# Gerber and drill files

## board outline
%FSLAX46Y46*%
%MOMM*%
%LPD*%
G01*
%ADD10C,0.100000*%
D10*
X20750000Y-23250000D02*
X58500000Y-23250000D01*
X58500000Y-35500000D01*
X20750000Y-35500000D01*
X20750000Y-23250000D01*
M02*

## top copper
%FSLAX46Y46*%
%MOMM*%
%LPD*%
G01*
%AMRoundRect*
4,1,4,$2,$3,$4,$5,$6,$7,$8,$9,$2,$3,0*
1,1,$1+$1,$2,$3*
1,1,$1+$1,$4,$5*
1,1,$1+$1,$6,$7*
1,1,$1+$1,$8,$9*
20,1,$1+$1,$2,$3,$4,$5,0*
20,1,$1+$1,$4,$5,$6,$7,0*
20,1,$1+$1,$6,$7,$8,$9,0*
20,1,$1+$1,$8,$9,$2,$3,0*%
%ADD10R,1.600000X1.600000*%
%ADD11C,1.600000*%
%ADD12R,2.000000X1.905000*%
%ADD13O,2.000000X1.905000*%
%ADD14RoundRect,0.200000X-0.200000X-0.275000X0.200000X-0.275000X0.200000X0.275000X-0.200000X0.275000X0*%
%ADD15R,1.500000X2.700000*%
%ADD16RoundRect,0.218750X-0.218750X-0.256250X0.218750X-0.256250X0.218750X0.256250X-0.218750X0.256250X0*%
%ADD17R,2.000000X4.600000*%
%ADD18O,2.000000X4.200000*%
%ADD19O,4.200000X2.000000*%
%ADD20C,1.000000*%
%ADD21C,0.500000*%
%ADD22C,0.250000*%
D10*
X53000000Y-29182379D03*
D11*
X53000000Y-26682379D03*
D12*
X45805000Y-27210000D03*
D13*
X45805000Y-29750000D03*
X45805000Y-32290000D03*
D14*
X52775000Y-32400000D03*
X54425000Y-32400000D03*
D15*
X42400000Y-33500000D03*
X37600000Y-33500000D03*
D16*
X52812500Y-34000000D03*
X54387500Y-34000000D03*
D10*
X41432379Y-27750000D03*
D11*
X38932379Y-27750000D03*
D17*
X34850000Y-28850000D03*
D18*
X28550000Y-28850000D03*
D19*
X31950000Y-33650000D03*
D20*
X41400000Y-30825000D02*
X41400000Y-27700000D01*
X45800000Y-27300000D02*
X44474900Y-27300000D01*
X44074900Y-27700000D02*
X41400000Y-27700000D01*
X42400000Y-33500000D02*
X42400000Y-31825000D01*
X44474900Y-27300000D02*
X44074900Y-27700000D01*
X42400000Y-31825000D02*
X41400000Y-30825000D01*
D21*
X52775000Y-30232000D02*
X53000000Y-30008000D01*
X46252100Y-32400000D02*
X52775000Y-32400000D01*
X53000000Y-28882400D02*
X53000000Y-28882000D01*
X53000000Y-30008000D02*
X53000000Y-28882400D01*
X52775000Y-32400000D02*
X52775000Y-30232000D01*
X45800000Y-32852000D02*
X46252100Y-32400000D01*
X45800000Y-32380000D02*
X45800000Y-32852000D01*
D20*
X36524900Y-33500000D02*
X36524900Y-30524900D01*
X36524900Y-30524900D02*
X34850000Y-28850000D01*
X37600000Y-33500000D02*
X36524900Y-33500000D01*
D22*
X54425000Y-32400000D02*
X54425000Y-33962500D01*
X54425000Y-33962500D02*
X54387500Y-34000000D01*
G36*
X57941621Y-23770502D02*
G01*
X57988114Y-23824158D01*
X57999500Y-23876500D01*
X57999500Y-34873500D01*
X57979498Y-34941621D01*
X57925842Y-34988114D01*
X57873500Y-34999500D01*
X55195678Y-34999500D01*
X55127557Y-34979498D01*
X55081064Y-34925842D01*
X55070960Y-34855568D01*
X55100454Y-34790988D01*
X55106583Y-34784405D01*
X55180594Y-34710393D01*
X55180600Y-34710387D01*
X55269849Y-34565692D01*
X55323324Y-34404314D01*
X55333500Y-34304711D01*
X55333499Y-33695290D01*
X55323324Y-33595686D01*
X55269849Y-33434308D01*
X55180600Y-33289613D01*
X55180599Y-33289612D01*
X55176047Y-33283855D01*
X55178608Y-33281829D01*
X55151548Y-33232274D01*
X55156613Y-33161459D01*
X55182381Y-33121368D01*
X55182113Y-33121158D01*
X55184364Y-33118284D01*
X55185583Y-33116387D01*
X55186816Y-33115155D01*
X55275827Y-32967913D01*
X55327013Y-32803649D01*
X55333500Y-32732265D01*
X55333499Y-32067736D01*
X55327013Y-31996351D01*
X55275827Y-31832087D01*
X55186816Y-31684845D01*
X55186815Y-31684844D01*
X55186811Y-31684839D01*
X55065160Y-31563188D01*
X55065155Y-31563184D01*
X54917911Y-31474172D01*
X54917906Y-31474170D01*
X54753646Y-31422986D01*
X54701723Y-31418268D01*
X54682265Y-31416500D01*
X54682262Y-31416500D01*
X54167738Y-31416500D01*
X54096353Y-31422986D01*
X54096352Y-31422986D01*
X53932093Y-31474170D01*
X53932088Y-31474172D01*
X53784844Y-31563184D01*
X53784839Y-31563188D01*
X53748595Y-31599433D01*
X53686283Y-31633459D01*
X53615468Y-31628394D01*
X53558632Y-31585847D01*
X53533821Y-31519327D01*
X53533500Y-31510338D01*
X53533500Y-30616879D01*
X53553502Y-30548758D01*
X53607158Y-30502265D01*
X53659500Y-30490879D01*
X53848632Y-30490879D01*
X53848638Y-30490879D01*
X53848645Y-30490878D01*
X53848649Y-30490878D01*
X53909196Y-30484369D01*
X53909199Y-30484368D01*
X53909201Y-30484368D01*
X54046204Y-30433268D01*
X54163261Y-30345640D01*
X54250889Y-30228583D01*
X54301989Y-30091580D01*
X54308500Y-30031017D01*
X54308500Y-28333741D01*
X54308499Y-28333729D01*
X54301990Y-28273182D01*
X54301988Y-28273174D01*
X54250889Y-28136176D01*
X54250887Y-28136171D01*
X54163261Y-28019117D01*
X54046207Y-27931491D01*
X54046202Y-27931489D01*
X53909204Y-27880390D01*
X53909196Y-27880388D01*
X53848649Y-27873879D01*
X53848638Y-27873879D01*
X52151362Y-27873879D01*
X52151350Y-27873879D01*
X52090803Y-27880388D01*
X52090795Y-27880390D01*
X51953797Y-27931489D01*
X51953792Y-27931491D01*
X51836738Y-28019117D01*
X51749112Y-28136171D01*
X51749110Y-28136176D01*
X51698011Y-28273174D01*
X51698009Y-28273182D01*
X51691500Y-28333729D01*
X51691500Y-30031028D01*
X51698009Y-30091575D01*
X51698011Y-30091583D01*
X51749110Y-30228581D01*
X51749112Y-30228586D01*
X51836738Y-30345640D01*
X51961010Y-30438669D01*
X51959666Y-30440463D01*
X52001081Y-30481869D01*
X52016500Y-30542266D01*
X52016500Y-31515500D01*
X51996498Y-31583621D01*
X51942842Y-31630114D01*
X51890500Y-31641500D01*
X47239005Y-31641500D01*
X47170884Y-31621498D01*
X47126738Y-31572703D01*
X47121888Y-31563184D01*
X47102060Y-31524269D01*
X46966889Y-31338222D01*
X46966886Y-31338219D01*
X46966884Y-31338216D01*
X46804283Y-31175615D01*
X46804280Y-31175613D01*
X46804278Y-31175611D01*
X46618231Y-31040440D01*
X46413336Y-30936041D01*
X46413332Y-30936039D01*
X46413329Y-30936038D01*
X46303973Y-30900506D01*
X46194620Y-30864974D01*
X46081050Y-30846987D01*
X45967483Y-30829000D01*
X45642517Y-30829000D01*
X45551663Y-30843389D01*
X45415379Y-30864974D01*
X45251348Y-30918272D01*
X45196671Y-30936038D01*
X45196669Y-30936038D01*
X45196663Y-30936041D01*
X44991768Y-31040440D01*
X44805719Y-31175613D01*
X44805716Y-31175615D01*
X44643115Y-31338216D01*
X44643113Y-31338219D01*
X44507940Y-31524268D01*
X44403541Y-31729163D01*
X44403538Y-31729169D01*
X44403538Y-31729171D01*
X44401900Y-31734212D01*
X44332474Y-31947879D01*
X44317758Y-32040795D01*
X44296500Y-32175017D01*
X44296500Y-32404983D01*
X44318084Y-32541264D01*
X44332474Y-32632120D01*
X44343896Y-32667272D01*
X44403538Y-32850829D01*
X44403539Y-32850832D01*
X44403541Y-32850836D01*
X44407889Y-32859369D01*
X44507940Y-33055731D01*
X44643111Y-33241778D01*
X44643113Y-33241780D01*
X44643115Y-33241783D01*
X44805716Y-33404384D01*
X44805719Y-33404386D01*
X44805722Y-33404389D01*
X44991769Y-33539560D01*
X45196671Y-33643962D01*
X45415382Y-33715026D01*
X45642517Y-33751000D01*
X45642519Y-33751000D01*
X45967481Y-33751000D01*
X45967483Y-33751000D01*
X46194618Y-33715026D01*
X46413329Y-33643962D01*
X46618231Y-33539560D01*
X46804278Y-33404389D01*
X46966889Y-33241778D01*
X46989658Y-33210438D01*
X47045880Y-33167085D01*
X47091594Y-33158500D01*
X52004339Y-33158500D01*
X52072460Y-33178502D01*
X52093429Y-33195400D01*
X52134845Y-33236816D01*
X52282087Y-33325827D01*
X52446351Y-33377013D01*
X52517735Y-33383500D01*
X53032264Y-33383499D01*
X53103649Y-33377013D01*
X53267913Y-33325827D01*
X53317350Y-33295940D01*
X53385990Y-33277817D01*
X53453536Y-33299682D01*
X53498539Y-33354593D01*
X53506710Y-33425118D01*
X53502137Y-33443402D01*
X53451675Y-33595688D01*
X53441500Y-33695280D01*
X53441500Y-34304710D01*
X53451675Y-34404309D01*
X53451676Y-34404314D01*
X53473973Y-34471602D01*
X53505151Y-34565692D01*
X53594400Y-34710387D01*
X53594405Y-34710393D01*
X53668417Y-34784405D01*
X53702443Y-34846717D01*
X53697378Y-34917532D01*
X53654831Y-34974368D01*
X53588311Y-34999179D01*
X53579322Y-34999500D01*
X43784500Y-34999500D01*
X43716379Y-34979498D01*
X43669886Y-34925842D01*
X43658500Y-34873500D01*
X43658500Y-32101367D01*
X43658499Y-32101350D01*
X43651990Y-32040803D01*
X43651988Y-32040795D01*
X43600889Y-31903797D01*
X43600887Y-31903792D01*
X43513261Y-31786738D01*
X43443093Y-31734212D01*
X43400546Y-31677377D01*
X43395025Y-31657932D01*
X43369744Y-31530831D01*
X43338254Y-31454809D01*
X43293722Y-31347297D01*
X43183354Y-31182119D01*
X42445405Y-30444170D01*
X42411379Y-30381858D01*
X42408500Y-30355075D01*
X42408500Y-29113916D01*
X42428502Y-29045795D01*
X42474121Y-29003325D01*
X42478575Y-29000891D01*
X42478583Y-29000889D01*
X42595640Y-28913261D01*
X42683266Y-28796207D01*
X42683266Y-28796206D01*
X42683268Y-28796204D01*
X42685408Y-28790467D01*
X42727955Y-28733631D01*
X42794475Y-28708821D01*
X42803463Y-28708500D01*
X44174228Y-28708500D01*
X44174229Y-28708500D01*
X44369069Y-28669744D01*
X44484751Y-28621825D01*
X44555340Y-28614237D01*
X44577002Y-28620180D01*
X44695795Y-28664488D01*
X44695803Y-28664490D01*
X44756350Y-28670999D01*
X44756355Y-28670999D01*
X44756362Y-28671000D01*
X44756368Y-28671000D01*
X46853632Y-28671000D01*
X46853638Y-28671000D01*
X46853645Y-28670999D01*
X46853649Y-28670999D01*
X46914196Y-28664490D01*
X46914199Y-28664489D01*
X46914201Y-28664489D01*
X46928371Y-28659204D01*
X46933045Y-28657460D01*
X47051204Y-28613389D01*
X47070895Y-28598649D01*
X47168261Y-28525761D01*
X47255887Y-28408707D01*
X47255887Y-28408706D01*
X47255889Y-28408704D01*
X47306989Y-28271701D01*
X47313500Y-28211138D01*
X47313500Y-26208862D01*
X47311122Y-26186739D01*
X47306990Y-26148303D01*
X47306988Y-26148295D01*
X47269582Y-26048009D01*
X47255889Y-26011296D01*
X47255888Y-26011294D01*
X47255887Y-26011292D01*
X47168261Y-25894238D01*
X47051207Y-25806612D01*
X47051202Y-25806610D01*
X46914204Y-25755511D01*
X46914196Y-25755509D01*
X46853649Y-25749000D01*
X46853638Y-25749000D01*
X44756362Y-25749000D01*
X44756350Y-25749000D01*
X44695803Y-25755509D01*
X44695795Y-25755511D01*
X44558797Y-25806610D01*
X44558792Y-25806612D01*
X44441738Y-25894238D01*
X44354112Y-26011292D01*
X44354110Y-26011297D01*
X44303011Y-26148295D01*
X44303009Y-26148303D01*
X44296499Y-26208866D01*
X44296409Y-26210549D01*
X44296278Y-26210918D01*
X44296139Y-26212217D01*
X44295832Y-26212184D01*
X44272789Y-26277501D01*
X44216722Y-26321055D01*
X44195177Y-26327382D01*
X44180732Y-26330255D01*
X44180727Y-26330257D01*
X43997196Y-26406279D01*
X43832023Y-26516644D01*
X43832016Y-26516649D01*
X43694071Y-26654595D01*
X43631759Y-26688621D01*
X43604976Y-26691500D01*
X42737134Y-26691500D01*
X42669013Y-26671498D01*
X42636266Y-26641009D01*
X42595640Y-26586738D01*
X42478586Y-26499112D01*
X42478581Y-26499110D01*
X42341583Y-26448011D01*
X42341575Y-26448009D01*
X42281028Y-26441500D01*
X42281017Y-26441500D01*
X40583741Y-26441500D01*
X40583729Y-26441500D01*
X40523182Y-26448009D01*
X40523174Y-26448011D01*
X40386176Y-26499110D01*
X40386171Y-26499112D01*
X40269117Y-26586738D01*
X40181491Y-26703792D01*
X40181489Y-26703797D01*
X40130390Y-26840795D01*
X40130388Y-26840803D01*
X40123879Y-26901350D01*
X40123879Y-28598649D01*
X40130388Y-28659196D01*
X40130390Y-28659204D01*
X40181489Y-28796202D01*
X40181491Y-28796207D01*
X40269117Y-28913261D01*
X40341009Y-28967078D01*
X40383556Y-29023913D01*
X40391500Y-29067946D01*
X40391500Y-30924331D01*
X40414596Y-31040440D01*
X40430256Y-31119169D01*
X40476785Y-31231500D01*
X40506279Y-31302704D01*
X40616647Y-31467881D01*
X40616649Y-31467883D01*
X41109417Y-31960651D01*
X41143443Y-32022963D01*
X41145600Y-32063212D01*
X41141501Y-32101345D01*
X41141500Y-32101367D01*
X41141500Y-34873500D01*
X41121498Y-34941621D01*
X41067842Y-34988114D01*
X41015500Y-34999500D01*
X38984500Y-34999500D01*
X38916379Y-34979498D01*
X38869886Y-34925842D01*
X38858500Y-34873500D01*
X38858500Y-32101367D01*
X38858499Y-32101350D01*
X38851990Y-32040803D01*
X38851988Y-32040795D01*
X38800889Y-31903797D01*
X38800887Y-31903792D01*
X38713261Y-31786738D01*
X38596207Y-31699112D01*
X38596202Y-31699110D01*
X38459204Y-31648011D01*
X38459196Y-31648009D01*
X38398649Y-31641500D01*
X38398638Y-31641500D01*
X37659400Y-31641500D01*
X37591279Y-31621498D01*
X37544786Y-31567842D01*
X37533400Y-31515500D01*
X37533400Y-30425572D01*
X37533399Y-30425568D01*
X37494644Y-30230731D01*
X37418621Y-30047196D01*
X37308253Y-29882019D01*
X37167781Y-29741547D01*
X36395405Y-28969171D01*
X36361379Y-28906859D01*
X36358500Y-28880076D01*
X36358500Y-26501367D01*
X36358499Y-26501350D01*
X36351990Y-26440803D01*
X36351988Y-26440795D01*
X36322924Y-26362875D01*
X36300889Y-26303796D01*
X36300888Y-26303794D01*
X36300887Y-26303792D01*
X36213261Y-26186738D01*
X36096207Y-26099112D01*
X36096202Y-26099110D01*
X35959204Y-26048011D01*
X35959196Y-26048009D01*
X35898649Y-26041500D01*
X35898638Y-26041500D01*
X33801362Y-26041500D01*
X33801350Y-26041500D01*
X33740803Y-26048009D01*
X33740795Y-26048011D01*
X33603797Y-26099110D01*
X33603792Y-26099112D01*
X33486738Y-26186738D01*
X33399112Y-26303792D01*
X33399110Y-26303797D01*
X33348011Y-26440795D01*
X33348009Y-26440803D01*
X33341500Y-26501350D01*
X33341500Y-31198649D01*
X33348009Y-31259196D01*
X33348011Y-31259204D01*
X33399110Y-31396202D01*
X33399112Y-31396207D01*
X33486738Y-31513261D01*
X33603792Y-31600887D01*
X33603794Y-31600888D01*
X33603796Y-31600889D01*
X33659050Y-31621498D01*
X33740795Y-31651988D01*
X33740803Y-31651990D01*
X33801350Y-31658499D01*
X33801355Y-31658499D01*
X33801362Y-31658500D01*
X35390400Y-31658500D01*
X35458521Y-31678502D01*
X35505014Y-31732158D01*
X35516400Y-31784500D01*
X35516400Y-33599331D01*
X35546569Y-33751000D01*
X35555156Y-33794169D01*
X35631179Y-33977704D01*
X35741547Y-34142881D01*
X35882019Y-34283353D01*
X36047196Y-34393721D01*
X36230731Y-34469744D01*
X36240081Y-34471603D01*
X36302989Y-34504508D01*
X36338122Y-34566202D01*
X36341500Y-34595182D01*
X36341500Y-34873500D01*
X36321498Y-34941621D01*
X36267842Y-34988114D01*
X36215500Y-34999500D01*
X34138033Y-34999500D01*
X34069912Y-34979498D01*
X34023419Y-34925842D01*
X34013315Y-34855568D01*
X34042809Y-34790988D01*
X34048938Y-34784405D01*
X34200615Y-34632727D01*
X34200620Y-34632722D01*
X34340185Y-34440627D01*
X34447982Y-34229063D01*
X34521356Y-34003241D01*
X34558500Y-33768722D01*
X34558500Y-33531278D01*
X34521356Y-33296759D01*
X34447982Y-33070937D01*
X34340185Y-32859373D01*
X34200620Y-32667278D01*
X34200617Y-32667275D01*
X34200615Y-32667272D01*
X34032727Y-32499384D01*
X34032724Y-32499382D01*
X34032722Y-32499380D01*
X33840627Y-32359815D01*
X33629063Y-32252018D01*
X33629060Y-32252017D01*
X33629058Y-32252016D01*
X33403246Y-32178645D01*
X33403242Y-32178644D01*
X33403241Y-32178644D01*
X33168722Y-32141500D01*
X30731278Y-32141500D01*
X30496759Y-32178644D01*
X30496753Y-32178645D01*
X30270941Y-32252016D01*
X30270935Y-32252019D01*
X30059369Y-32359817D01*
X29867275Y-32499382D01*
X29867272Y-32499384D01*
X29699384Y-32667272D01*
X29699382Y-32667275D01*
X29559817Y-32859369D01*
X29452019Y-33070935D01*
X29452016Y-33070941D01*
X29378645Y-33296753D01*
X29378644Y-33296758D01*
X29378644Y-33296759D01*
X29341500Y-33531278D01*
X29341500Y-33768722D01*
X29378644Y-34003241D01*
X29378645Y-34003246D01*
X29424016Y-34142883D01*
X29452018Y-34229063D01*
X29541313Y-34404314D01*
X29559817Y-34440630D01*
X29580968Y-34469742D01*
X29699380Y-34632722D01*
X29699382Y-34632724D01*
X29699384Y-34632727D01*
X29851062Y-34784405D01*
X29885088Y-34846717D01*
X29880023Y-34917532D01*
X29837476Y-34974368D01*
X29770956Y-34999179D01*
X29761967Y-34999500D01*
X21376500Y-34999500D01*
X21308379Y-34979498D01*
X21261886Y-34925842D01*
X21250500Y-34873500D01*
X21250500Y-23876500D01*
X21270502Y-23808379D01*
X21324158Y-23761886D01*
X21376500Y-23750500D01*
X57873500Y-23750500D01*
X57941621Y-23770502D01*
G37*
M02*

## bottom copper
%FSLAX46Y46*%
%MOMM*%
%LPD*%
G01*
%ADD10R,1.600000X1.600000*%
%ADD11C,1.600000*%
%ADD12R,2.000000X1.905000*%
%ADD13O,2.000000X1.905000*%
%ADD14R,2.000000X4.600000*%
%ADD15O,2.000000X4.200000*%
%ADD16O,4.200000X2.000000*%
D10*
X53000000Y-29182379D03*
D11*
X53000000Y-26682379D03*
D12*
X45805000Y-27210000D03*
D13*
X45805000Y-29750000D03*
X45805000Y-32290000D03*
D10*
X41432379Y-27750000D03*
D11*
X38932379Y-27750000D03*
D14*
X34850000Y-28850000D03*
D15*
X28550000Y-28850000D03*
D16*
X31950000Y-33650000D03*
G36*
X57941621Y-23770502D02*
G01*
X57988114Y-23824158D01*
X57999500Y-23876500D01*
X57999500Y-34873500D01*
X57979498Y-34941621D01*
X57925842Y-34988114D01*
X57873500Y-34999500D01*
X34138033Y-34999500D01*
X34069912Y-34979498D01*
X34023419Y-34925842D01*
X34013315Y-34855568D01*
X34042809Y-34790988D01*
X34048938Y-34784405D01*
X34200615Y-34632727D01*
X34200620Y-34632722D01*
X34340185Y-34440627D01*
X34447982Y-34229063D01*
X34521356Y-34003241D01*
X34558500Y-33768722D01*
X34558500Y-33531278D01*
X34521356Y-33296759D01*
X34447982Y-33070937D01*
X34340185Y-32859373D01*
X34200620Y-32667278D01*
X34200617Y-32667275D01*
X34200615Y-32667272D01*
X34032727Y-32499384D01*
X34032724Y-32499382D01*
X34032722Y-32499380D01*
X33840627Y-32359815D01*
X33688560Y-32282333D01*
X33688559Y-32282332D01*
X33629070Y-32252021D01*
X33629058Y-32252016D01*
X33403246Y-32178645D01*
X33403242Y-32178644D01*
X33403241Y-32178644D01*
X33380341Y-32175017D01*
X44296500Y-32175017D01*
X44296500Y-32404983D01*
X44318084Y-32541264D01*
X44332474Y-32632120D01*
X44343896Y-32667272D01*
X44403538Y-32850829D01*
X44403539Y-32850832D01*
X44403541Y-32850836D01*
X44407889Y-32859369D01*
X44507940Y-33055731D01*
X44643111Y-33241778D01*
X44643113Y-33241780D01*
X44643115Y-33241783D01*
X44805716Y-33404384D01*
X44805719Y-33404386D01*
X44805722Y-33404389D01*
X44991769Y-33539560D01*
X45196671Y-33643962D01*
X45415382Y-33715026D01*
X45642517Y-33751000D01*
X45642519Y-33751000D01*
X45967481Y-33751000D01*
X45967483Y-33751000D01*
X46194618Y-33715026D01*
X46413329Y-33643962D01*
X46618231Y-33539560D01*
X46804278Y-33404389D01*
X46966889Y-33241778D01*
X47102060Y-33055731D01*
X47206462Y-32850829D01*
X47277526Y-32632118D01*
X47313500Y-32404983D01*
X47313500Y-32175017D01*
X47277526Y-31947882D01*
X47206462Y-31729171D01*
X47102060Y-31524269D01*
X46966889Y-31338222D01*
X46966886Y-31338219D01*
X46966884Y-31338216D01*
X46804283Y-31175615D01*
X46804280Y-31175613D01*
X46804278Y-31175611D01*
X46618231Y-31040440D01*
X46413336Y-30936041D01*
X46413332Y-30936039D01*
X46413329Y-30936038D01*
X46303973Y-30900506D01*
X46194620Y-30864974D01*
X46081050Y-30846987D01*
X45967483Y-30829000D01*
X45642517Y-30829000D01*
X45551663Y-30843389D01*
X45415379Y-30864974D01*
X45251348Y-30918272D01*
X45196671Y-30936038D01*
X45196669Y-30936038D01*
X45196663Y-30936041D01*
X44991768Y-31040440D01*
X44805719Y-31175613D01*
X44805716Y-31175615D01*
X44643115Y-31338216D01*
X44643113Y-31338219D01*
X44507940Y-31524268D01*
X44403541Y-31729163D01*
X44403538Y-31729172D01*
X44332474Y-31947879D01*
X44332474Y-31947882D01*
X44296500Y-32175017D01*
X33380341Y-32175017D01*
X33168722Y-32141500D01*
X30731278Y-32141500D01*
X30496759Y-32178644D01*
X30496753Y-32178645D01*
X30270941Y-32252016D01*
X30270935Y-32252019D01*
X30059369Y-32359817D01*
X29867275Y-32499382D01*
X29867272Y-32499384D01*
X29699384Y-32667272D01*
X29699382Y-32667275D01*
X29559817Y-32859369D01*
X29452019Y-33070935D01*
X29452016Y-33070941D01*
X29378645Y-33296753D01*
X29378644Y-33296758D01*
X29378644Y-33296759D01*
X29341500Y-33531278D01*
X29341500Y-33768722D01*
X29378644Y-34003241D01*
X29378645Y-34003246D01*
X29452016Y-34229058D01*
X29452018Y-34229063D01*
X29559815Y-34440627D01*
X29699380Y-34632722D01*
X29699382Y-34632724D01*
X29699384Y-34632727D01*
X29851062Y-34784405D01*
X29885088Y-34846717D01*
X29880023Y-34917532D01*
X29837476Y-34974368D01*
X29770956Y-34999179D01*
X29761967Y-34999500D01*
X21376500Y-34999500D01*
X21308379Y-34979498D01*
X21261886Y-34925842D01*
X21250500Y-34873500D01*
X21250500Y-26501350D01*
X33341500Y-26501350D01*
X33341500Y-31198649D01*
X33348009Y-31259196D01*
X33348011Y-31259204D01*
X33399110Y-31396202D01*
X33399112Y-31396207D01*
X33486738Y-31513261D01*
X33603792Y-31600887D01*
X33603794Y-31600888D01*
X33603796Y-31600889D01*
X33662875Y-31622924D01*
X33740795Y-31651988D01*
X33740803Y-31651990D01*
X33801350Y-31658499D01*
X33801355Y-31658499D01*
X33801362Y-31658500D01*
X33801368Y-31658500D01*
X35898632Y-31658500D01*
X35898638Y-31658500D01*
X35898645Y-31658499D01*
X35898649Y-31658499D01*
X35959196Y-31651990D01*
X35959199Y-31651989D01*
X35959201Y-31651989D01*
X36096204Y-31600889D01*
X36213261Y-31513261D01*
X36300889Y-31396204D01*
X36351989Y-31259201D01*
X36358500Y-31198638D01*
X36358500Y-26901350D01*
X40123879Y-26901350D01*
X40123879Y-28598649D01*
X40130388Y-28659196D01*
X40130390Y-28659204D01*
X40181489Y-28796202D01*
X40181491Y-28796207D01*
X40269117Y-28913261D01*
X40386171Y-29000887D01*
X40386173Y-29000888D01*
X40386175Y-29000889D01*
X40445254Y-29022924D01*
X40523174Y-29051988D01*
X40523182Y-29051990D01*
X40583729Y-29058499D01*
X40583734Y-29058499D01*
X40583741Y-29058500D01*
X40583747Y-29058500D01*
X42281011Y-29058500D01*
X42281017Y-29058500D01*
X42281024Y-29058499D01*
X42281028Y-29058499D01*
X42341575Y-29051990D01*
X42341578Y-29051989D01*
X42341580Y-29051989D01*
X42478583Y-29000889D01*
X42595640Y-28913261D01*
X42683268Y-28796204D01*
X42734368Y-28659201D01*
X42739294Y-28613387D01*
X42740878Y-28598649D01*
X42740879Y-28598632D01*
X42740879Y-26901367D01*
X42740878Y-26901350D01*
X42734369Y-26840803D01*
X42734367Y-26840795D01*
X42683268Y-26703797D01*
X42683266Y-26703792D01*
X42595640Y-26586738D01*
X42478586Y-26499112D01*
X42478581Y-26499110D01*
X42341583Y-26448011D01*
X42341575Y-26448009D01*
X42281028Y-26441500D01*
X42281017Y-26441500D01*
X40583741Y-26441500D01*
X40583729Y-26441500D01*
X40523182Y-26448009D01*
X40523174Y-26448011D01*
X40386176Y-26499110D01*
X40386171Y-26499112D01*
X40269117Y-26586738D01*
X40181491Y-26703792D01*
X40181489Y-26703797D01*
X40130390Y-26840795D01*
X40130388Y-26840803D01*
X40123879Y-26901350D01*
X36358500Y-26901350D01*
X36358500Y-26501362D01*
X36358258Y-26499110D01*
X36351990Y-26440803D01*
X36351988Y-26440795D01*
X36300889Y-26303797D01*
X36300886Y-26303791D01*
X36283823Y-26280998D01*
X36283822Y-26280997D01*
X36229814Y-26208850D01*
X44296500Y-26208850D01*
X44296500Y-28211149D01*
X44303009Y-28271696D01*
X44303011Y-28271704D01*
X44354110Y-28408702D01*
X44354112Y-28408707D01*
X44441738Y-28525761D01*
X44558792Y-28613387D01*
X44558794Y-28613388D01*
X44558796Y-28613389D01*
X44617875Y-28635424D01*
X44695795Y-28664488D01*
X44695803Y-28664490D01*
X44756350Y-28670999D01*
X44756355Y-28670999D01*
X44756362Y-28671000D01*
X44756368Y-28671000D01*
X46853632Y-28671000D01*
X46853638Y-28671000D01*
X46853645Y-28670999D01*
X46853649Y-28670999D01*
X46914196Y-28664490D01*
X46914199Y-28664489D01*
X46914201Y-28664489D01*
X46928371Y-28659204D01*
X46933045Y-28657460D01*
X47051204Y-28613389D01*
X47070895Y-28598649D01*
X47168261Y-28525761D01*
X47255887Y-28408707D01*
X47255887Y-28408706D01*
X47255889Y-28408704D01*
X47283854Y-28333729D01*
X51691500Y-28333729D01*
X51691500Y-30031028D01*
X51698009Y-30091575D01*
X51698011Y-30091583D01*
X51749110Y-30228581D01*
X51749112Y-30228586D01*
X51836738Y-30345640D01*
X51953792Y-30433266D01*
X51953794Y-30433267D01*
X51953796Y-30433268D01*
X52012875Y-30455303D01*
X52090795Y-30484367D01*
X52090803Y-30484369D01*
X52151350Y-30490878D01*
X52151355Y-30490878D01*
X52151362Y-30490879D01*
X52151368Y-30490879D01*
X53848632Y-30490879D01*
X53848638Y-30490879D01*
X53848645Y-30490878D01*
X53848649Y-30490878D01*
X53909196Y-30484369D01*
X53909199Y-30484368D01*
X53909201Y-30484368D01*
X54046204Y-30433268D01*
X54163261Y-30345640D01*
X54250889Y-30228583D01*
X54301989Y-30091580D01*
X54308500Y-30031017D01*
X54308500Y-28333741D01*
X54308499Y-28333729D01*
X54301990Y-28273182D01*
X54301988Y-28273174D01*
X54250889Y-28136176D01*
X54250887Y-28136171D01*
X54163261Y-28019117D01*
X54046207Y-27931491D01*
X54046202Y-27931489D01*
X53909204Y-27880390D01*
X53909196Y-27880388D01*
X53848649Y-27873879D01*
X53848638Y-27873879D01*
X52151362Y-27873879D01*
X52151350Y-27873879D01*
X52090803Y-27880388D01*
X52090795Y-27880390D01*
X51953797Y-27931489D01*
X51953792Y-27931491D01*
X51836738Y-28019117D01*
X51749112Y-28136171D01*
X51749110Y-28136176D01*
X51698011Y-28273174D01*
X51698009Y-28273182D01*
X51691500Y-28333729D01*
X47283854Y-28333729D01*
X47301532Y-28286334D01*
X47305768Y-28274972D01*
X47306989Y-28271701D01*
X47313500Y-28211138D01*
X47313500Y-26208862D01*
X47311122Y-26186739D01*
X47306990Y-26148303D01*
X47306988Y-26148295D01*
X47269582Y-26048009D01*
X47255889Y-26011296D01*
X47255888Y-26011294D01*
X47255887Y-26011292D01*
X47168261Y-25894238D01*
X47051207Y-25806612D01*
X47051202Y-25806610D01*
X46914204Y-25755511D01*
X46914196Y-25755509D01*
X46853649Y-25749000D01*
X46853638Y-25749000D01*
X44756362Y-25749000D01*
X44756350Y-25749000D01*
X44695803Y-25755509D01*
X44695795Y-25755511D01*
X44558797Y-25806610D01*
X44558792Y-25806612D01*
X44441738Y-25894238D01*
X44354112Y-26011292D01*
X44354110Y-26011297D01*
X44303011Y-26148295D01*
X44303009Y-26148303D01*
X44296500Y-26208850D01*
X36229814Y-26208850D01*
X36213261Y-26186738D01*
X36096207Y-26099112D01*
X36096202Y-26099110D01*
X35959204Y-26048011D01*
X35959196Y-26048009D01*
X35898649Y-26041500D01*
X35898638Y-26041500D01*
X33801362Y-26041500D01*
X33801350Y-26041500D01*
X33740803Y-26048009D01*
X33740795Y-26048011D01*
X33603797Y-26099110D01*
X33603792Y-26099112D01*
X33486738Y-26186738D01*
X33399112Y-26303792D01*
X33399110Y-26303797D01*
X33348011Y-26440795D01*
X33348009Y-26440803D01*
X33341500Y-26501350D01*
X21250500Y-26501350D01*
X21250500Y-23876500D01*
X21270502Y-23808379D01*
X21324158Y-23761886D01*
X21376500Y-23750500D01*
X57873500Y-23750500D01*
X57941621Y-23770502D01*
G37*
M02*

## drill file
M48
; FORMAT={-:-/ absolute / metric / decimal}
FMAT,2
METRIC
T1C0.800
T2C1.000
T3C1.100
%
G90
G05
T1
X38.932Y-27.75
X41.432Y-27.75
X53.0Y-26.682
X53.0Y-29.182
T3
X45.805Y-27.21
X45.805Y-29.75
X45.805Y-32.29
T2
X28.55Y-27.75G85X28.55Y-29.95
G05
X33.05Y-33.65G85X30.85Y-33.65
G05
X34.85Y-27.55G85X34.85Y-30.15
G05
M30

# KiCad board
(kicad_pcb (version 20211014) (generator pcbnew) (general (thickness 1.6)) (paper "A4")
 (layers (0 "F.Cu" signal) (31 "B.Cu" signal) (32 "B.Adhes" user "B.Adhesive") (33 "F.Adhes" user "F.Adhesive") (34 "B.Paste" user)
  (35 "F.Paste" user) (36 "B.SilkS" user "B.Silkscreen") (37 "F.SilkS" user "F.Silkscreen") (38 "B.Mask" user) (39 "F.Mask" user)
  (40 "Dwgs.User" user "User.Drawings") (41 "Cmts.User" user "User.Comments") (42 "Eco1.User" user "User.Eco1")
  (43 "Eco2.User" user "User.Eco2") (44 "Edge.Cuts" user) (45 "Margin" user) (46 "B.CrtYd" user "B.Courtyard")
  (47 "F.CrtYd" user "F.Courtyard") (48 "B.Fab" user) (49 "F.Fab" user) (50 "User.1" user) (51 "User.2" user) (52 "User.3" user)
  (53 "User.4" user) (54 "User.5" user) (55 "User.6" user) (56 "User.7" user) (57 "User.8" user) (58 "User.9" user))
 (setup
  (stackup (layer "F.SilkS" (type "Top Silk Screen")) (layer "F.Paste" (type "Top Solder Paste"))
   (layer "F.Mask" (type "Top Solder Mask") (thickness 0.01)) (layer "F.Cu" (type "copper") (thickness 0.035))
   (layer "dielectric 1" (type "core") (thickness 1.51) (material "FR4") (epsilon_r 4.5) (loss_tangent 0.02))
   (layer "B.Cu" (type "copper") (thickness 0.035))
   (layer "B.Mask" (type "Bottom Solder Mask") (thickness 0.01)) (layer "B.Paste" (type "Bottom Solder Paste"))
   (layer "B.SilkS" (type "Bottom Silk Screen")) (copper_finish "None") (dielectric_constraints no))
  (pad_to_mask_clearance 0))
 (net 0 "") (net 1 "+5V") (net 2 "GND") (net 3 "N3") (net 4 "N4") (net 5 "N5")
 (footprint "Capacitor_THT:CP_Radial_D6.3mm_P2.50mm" (layer "F.Cu") (at 53 29.182379 90)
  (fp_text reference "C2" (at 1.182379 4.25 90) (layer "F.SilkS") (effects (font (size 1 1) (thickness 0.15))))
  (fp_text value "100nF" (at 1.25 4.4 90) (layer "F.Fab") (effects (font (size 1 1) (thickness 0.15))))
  (pad "1" thru_hole rect (at 0 0 90) (size 1.6 1.6) (drill 0.8) (layers *.Cu *.Mask) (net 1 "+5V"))
  (pad "2" thru_hole circle (at 2.5 0 90) (size 1.6 1.6) (drill 0.8) (layers *.Cu *.Mask) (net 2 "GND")))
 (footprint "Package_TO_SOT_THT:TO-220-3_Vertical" (layer "F.Cu") (at 45.805 27.21 -90)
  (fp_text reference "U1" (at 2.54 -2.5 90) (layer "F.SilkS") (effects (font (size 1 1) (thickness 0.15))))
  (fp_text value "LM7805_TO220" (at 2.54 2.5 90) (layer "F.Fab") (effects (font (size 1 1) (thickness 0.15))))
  (pad "1" thru_hole rect (at 0 0 270) (size 1.905 2) (drill 1.1) (layers *.Cu *.Mask) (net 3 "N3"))
  (pad "2" thru_hole oval (at 2.54 0 270) (size 1.905 2) (drill 1.1) (layers *.Cu *.Mask) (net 2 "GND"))
  (pad "3" thru_hole oval (at 5.08 0 270) (size 1.905 2) (drill 1.1) (layers *.Cu *.Mask) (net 1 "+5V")))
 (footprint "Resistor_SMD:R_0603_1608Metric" (layer "F.Cu") (at 53.6 32.4)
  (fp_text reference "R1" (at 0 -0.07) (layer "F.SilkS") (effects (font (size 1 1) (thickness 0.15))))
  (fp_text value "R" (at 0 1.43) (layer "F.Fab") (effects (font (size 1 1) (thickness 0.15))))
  (pad "1" smd roundrect (at -0.825 0) (size 0.8 0.95) (layers "F.Cu" "F.Paste" "F.Mask") (roundrect_rratio 0.25) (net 1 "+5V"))
  (pad "2" smd roundrect (at 0.825 0) (size 0.8 0.95) (layers "F.Cu" "F.Paste" "F.Mask") (roundrect_rratio 0.25) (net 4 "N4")))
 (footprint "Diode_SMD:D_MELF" (layer "F.Cu") (at 40 33.5 180)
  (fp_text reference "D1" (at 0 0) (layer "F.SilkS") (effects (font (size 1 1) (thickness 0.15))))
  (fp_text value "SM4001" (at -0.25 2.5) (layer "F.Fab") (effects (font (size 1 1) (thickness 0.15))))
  (pad "1" smd rect (at -2.4 0 180) (size 1.5 2.7) (layers "F.Cu" "F.Paste" "F.Mask") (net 3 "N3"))
  (pad "2" smd rect (at 2.4 0 180) (size 1.5 2.7) (layers "F.Cu" "F.Paste" "F.Mask") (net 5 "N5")))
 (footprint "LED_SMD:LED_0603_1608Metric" (layer "F.Cu") (at 53.6 34)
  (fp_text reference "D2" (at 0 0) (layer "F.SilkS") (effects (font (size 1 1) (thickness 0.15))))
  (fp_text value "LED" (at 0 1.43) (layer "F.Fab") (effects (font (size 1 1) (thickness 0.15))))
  (pad "1" smd roundrect (at -0.7875 0) (size 0.875 0.95) (layers "F.Cu" "F.Paste" "F.Mask") (roundrect_rratio 0.25) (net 2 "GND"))
  (pad "2" smd roundrect (at 0.7875 0) (size 0.875 0.95) (layers "F.Cu" "F.Paste" "F.Mask") (roundrect_rratio 0.25) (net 4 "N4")))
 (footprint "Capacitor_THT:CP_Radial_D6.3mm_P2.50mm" (layer "F.Cu") (at 41.432379 27.75 180)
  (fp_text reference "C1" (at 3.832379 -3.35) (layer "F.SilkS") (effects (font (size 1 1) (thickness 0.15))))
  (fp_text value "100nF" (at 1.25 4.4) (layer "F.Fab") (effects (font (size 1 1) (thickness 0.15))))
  (pad "1" thru_hole rect (at 0 0 180) (size 1.6 1.6) (drill 0.8) (layers *.Cu *.Mask) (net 3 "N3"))
  (pad "2" thru_hole circle (at 2.5 0 180) (size 1.6 1.6) (drill 0.8) (layers *.Cu *.Mask) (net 2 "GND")))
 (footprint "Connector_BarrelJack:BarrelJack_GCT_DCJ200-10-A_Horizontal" (layer "F.Cu") (at 34.85 28.85 -90)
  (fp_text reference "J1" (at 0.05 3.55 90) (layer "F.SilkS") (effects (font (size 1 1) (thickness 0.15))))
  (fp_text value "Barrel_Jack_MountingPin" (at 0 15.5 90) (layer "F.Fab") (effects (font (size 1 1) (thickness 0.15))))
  (pad "1" thru_hole rect (at 0 0 270) (size 4.6 2) (drill oval 3.6 1) (layers *.Cu *.Mask) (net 5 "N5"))
  (pad "2" thru_hole oval (at 0 6.3 270) (size 4.2 2) (drill oval 3.2 1) (layers *.Cu *.Mask) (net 2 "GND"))
  (pad "3" thru_hole oval (at 4.8 2.9 270) (size 2 4.2) (drill oval 1 3.2) (layers *.Cu *.Mask)))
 (gr_rect (start 58.5 23.25) (end 20.75 35.5) (layer "Edge.Cuts") (width 0.1) (fill none))
 (segment (start 41.4 30.825) (end 41.4 27.7) (width 1) (layer "F.Cu") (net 3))
 (segment (start 45.8 27.3) (end 44.4749 27.3) (width 1) (layer "F.Cu") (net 3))
 (segment (start 44.0749 27.7) (end 41.4 27.7) (width 1) (layer "F.Cu") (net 3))
 (segment (start 42.4 33.5) (end 42.4 31.825) (width 1) (layer "F.Cu") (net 3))
 (segment (start 44.4749 27.3) (end 44.0749 27.7) (width 1) (layer "F.Cu") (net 3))
 (segment (start 42.4 31.825) (end 41.4 30.825) (width 1) (layer "F.Cu") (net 3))
 (segment (start 52.775 30.232) (end 53 30.008) (width 0.5) (layer "F.Cu") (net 1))
 (segment (start 46.2521 32.4) (end 52.775 32.4) (width 0.5) (layer "F.Cu") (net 1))
 (segment (start 53 28.8824) (end 53 28.882) (width 0.5) (layer "F.Cu") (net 1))
 (segment (start 53 30.008) (end 53 28.8824) (width 0.5) (layer "F.Cu") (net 1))
 (segment (start 52.775 32.4) (end 52.775 30.232) (width 0.5) (layer "F.Cu") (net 1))
 (segment (start 45.8 32.852) (end 46.2521 32.4) (width 0.5) (layer "F.Cu") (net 1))
 (segment (start 45.8 32.38) (end 45.8 32.852) (width 0.5) (layer "F.Cu") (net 1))
 (segment (start 36.5249 33.5) (end 36.5249 30.5249) (width 1) (layer "F.Cu") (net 5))
 (segment (start 36.5249 30.5249) (end 34.85 28.85) (width 1) (layer "F.Cu") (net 5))
 (segment (start 37.6 33.5) (end 36.5249 33.5) (width 1) (layer "F.Cu") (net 5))
 (segment (start 54.425 32.4) (end 54.425 33.9625) (width 0.25) (layer "F.Cu") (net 4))
 (segment (start 54.425 33.9625) (end 54.3875 34) (width 0.25) (layer "F.Cu") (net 4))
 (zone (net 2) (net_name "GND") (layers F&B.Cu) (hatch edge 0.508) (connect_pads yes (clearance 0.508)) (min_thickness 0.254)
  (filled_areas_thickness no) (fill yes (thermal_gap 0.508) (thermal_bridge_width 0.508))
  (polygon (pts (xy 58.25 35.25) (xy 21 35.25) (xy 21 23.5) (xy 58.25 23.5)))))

